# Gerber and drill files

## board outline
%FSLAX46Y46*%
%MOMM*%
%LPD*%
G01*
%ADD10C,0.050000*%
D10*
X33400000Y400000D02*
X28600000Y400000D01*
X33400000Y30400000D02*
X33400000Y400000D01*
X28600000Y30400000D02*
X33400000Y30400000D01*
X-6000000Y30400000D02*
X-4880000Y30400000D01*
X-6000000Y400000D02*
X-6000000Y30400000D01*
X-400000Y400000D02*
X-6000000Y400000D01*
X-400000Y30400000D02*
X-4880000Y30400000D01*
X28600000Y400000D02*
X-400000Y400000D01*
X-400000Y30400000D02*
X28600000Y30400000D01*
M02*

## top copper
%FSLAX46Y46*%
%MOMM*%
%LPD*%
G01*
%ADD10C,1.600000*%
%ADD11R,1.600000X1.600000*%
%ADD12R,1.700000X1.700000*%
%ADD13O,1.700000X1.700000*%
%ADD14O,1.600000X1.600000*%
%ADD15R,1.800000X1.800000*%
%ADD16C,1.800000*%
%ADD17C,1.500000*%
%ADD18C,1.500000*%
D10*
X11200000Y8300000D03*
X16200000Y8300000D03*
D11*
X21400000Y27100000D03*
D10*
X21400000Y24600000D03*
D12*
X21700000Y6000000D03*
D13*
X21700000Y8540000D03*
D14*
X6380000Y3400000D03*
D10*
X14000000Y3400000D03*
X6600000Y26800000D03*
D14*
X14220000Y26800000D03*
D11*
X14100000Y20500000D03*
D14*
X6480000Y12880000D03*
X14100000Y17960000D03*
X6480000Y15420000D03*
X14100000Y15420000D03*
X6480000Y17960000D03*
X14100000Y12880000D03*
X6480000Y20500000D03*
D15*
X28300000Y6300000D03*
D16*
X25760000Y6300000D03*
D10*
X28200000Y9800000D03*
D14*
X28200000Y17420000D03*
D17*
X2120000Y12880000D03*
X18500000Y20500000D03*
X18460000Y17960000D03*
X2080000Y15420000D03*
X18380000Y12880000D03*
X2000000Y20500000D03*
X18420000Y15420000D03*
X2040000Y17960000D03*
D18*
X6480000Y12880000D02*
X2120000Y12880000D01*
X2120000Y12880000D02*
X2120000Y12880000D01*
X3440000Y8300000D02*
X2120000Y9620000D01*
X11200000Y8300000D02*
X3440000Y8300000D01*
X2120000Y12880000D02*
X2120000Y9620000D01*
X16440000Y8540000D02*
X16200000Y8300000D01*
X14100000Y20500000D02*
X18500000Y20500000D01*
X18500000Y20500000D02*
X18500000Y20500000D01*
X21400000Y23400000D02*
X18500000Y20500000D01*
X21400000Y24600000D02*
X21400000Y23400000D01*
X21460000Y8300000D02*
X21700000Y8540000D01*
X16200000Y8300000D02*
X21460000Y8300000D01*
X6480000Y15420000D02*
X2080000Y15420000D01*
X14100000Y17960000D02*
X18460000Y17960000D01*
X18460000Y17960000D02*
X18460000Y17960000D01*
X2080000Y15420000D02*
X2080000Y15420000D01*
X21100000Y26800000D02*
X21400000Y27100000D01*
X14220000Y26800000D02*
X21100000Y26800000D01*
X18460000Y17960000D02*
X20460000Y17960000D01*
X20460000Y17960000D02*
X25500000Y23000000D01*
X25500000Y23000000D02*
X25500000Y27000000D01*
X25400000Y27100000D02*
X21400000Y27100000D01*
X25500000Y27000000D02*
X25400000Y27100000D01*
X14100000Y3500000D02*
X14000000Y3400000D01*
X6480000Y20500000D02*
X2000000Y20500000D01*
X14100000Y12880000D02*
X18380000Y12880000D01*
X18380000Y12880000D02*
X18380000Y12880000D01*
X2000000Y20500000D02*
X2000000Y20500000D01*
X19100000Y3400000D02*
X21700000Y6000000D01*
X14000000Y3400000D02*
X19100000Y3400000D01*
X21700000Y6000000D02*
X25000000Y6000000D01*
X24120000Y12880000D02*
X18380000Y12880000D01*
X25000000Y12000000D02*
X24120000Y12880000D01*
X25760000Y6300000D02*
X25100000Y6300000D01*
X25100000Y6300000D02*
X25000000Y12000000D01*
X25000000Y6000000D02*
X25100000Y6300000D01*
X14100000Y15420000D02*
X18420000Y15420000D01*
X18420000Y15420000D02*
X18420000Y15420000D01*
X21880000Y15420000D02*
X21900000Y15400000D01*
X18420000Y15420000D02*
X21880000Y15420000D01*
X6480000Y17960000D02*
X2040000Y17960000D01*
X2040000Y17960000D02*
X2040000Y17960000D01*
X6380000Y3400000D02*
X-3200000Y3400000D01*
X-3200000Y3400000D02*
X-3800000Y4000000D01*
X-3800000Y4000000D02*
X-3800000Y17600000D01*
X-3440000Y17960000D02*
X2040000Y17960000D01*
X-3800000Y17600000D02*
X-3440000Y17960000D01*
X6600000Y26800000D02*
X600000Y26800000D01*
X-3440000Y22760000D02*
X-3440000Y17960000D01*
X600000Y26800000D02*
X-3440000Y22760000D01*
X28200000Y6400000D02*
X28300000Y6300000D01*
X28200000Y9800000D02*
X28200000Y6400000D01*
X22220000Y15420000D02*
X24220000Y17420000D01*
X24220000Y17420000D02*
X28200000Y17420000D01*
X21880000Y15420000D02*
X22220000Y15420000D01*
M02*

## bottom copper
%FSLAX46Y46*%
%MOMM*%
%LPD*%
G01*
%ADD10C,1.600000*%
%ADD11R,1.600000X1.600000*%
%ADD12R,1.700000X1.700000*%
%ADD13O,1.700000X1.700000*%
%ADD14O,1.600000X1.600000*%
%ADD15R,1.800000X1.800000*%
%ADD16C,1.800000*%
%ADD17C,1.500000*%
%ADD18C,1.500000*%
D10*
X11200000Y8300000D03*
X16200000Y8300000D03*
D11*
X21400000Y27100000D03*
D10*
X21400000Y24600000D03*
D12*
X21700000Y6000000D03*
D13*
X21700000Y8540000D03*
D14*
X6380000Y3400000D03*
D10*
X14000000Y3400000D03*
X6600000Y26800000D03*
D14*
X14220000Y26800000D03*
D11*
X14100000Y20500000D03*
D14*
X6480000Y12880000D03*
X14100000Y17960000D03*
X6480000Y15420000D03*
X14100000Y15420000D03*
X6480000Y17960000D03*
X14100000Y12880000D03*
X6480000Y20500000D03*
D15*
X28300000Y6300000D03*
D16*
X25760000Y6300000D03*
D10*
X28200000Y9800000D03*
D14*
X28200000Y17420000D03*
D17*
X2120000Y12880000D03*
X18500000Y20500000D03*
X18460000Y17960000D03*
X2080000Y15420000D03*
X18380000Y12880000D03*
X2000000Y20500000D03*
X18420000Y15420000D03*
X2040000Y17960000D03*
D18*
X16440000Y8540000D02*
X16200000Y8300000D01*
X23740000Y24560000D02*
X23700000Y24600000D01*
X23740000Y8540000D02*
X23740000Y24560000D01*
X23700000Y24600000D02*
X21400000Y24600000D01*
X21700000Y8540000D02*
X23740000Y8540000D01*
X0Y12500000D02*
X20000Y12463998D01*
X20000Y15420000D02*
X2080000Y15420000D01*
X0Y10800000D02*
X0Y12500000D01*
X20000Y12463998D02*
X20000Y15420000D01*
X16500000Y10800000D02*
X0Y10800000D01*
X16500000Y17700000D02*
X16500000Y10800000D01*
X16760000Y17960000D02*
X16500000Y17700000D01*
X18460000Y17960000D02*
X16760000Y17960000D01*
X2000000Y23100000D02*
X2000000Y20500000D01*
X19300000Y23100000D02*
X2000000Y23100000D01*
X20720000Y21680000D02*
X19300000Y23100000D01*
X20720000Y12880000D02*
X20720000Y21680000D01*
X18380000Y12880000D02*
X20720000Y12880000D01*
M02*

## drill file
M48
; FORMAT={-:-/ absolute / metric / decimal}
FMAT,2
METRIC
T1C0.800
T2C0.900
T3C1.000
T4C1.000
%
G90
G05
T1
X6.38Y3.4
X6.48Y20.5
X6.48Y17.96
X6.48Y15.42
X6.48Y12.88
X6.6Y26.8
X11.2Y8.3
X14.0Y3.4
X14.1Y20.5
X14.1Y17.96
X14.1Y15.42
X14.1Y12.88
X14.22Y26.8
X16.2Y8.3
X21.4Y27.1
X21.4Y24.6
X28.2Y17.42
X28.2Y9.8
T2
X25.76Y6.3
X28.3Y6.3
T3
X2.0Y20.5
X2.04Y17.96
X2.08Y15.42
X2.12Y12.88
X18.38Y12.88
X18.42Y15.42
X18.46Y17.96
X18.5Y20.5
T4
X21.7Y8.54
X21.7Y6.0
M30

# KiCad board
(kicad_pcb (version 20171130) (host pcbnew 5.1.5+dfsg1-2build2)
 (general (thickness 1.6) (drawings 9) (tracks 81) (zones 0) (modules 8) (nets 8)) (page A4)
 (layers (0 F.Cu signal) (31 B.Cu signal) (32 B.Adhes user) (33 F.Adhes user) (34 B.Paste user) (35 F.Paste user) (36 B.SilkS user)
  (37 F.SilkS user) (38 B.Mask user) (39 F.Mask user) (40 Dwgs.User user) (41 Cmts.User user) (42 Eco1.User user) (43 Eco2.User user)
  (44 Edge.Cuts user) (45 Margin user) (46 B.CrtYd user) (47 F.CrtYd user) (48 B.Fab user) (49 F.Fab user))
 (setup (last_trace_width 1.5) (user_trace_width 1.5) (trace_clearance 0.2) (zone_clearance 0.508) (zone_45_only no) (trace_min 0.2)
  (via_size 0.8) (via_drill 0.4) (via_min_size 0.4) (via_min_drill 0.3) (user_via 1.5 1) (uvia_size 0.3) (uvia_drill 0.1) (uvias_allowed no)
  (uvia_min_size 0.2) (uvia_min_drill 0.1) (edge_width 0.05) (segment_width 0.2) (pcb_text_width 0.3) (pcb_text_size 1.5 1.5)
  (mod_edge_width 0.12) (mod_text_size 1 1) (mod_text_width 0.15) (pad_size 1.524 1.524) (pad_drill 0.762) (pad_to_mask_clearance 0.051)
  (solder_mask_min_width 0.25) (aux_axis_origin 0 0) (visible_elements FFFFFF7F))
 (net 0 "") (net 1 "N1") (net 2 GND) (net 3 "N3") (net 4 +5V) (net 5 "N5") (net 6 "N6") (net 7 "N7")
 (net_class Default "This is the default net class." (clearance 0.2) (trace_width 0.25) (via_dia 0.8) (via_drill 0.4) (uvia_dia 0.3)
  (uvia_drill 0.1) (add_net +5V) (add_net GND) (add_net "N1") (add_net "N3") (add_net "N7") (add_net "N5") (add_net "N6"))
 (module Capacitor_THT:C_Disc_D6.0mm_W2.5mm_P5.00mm (layer F.Cu) (at 11.2 -8.3)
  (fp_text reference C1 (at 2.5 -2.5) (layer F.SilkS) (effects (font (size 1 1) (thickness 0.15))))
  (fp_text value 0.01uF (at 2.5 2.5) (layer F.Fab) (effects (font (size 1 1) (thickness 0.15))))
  (pad 1 thru_hole circle (at 0 0) (size 1.6 1.6) (drill 0.8) (layers *.Cu *.Mask) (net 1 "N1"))
  (pad 2 thru_hole circle (at 5 0) (size 1.6 1.6) (drill 0.8) (layers *.Cu *.Mask) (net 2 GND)))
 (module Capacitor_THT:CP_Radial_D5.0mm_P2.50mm (layer F.Cu) (at 21.4 -27.1 270)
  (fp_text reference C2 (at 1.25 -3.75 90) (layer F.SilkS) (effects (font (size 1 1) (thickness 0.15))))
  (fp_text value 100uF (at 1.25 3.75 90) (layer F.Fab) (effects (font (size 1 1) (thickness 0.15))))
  (pad 1 thru_hole rect (at 0 0 270) (size 1.6 1.6) (drill 0.8) (layers *.Cu *.Mask) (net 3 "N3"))
  (pad 2 thru_hole circle (at 2.5 0 270) (size 1.6 1.6) (drill 0.8) (layers *.Cu *.Mask) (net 2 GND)))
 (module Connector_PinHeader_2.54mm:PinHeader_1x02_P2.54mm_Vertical (layer F.Cu) (at 21.7 -6 180)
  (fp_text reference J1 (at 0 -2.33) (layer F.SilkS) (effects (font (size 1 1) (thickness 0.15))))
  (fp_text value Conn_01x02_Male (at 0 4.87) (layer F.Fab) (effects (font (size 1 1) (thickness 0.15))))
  (pad 1 thru_hole rect (at 0 0 180) (size 1.7 1.7) (drill 1) (layers *.Cu *.Mask) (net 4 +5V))
  (pad 2 thru_hole oval (at 0 2.54 180) (size 1.7 1.7) (drill 1) (layers *.Cu *.Mask) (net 2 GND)))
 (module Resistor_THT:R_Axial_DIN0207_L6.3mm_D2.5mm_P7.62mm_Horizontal (layer F.Cu) (at 14 -3.4 180)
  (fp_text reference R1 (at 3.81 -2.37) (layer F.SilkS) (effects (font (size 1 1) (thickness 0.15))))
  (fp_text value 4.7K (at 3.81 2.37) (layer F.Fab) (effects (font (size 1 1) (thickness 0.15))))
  (pad 2 thru_hole oval (at 7.62 0 180) (size 1.6 1.6) (drill 0.8) (layers *.Cu *.Mask) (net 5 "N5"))
  (pad 1 thru_hole circle (at 0 0 180) (size 1.6 1.6) (drill 0.8) (layers *.Cu *.Mask) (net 4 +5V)))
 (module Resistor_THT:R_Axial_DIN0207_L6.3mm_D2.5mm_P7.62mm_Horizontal (layer F.Cu) (at 6.6 -26.8)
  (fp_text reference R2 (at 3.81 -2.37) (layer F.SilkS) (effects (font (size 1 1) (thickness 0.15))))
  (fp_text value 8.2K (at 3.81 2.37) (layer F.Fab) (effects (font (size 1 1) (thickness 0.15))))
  (pad 1 thru_hole circle (at 0 0) (size 1.6 1.6) (drill 0.8) (layers *.Cu *.Mask) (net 5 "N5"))
  (pad 2 thru_hole oval (at 7.62 0) (size 1.6 1.6) (drill 0.8) (layers *.Cu *.Mask) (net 3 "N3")))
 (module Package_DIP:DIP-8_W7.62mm (layer B.Cu) (at 14.1 -20.5 180)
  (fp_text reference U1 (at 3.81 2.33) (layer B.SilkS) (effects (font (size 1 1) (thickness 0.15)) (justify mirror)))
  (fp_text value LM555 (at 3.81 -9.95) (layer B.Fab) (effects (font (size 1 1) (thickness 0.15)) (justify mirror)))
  (pad 1 thru_hole rect (at 0 0 180) (size 1.6 1.6) (drill 0.8) (layers *.Cu *.Mask) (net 2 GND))
  (pad 5 thru_hole oval (at 7.62 -7.62 180) (size 1.6 1.6) (drill 0.8) (layers *.Cu *.Mask) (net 1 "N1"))
  (pad 2 thru_hole oval (at 0 -2.54 180) (size 1.6 1.6) (drill 0.8) (layers *.Cu *.Mask) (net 3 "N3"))
  (pad 6 thru_hole oval (at 7.62 -5.08 180) (size 1.6 1.6) (drill 0.8) (layers *.Cu *.Mask) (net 3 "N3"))
  (pad 3 thru_hole oval (at 0 -5.08 180) (size 1.6 1.6) (drill 0.8) (layers *.Cu *.Mask) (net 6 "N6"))
  (pad 7 thru_hole oval (at 7.62 -2.54 180) (size 1.6 1.6) (drill 0.8) (layers *.Cu *.Mask) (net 5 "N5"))
  (pad 4 thru_hole oval (at 0 -7.62 180) (size 1.6 1.6) (drill 0.8) (layers *.Cu *.Mask) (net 4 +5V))
  (pad 8 thru_hole oval (at 7.62 0 180) (size 1.6 1.6) (drill 0.8) (layers *.Cu *.Mask) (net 4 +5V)))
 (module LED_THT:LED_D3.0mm (layer F.Cu) (at 28.3 -6.3 180)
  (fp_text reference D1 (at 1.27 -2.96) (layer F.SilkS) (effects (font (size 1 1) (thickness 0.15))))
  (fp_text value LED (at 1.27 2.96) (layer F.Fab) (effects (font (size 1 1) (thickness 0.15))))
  (pad 1 thru_hole rect (at 0 0 180) (size 1.8 1.8) (drill 0.9) (layers *.Cu *.Mask) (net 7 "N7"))
  (pad 2 thru_hole circle (at 2.54 0 180) (size 1.8 1.8) (drill 0.9) (layers *.Cu *.Mask) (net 4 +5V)))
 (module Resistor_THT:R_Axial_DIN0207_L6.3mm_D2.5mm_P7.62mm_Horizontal (layer F.Cu) (at 28.2 -9.8 90)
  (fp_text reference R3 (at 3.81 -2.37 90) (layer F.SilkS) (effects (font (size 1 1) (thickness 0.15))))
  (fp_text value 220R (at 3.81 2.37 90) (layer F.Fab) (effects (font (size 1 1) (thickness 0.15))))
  (pad 1 thru_hole circle (at 0 0 90) (size 1.6 1.6) (drill 0.8) (layers *.Cu *.Mask) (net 7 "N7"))
  (pad 2 thru_hole oval (at 7.62 0 90) (size 1.6 1.6) (drill 0.8) (layers *.Cu *.Mask) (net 6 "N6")))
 (gr_line (start 33.4 -0.4) (end 28.6 -0.4) (layer Edge.Cuts) (width 0.05))
 (gr_line (start 33.4 -30.4) (end 33.4 -0.4) (layer Edge.Cuts) (width 0.05))
 (gr_line (start 28.6 -30.4) (end 33.4 -30.4) (layer Edge.Cuts) (width 0.05))
 (gr_line (start -6 -30.4) (end -4.88 -30.4) (layer Edge.Cuts) (width 0.05))
 (gr_line (start -6 -0.4) (end -6 -30.4) (layer Edge.Cuts) (width 0.05))
 (gr_line (start -0.4 -0.4) (end -6 -0.4) (layer Edge.Cuts) (width 0.05))
 (gr_line (start -0.4 -30.4) (end -4.88 -30.4) (layer Edge.Cuts) (width 0.05))
 (gr_line (start 28.6 -0.4) (end -0.4 -0.4) (layer Edge.Cuts) (width 0.05))
 (gr_line (start -0.4 -30.4) (end 28.6 -30.4) (layer Edge.Cuts) (width 0.05))
 (segment (start 6.48 -12.88) (end 2.12 -12.88) (width 1.5) (layer F.Cu) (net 1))
 (segment (start 2.12 -12.88) (end 2.12 -12.88) (width 1.5) (layer F.Cu) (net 1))
 (via (at 2.12 -12.88) (size 1.5) (drill 1) (layers F.Cu B.Cu) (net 1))
 (segment (start 3.44 -8.3) (end 2.12 -9.62) (width 1.5) (layer F.Cu) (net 1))
 (segment (start 11.2 -8.3) (end 3.44 -8.3) (width 1.5) (layer F.Cu) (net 1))
 (segment (start 2.12 -12.88) (end 2.12 -9.62) (width 1.5) (layer F.Cu) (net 1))
 (segment (start 16.44 -8.54) (end 16.2 -8.3) (width 1.5) (layer B.Cu) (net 2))
 (segment (start 16.44 -8.54) (end 16.2 -8.3) (width 1.5) (layer F.Cu) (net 2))
 (segment (start 14.1 -20.5) (end 18.5 -20.5) (width 1.5) (layer F.Cu) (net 2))
 (segment (start 18.5 -20.5) (end 18.5 -20.5) (width 1.5) (layer F.Cu) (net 2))
 (via (at 18.5 -20.5) (size 1.5) (drill 1) (layers F.Cu B.Cu) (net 2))
 (segment (start 21.4 -23.4) (end 18.5 -20.5) (width 1.5) (layer F.Cu) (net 2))
 (segment (start 21.4 -24.6) (end 21.4 -23.4) (width 1.5) (layer F.Cu) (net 2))
 (segment (start 21.46 -8.3) (end 21.7 -8.54) (width 1.5) (layer F.Cu) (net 2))
 (segment (start 16.2 -8.3) (end 21.46 -8.3) (width 1.5) (layer F.Cu) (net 2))
 (segment (start 23.74 -24.56) (end 23.7 -24.6) (width 1.5) (layer B.Cu) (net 2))
 (segment (start 23.74 -8.54) (end 23.74 -24.56) (width 1.5) (layer B.Cu) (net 2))
 (segment (start 23.7 -24.6) (end 21.4 -24.6) (width 1.5) (layer B.Cu) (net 2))
 (segment (start 21.7 -8.54) (end 23.74 -8.54) (width 1.5) (layer B.Cu) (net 2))
 (segment (start 6.48 -15.42) (end 2.08 -15.42) (width 1.5) (layer F.Cu) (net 3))
 (segment (start 14.1 -17.96) (end 18.46 -17.96) (width 1.5) (layer F.Cu) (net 3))
 (segment (start 18.46 -17.96) (end 18.46 -17.96) (width 1.5) (layer F.Cu) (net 3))
 (via (at 18.46 -17.96) (size 1.5) (drill 1) (layers F.Cu B.Cu) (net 3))
 (segment (start 2.08 -15.42) (end 2.08 -15.42) (width 1.5) (layer F.Cu) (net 3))
 (via (at 2.08 -15.42) (size 1.5) (drill 1) (layers F.Cu B.Cu) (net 3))
 (segment (start 21.1 -26.8) (end 21.4 -27.1) (width 1.5) (layer F.Cu) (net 3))
 (segment (start 14.22 -26.8) (end 21.1 -26.8) (width 1.5) (layer F.Cu) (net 3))
 (segment (start 18.46 -17.96) (end 20.46 -17.96) (width 1.5) (layer F.Cu) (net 3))
 (segment (start 20.46 -17.96) (end 25.5 -23) (width 1.5) (layer F.Cu) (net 3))
 (segment (start 25.5 -23) (end 25.5 -27) (width 1.5) (layer F.Cu) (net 3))
 (segment (start 25.4 -27.1) (end 21.4 -27.1) (width 1.5) (layer F.Cu) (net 3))
 (segment (start 25.5 -27) (end 25.4 -27.1) (width 1.5) (layer F.Cu) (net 3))
 (segment (start 0 -12.5) (end 0.02 -12.463998) (width 1.5) (layer B.Cu) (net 3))
 (segment (start 0.02 -15.42) (end 2.08 -15.42) (width 1.5) (layer B.Cu) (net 3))
 (segment (start 0 -10.8) (end 0 -12.5) (width 1.5) (layer B.Cu) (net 3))
 (segment (start 0.02 -12.463998) (end 0.02 -15.42) (width 1.5) (layer B.Cu) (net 3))
 (segment (start 16.5 -10.8) (end 0 -10.8) (width 1.5) (layer B.Cu) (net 3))
 (segment (start 16.5 -17.7) (end 16.5 -10.8) (width 1.5) (layer B.Cu) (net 3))
 (segment (start 16.76 -17.96) (end 16.5 -17.7) (width 1.5) (layer B.Cu) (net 3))
 (segment (start 18.46 -17.96) (end 16.76 -17.96) (width 1.5) (layer B.Cu) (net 3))
 (segment (start 14.1 -3.5) (end 14 -3.4) (width 1.5) (layer F.Cu) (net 4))
 (segment (start 6.48 -20.5) (end 2 -20.5) (width 1.5) (layer F.Cu) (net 4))
 (segment (start 14.1 -12.88) (end 18.38 -12.88) (width 1.5) (layer F.Cu) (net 4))
 (segment (start 18.38 -12.88) (end 18.38 -12.88) (width 1.5) (layer F.Cu) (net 4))
 (via (at 18.38 -12.88) (size 1.5) (drill 1) (layers F.Cu B.Cu) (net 4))
 (segment (start 2 -20.5) (end 2 -20.5) (width 1.5) (layer F.Cu) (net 4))
 (via (at 2 -20.5) (size 1.5) (drill 1) (layers F.Cu B.Cu) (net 4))
 (segment (start 19.1 -3.4) (end 21.7 -6) (width 1.5) (layer F.Cu) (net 4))
 (segment (start 14 -3.4) (end 19.1 -3.4) (width 1.5) (layer F.Cu) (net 4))
 (segment (start 21.7 -6) (end 25 -6) (width 1.5) (layer F.Cu) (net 4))
 (segment (start 24.12 -12.88) (end 18.38 -12.88) (width 1.5) (layer F.Cu) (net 4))
 (segment (start 25 -12) (end 24.12 -12.88) (width 1.5) (layer F.Cu) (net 4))
 (segment (start 2 -23.1) (end 2 -20.5) (width 1.5) (layer B.Cu) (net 4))
 (segment (start 19.3 -23.1) (end 2 -23.1) (width 1.5) (layer B.Cu) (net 4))
 (segment (start 20.72 -21.68) (end 19.3 -23.1) (width 1.5) (layer B.Cu) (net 4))
 (segment (start 20.72 -12.88) (end 20.72 -21.68) (width 1.5) (layer B.Cu) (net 4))
 (segment (start 18.38 -12.88) (end 20.72 -12.88) (width 1.5) (layer B.Cu) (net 4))
 (segment (start 25.76 -6.3) (end 25.1 -6.3) (width 1.5) (layer F.Cu) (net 4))
 (segment (start 25.1 -6.3) (end 25 -12) (width 1.5) (layer F.Cu) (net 4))
 (segment (start 25 -6) (end 25.1 -6.3) (width 1.5) (layer F.Cu) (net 4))
 (segment (start 14.1 -15.42) (end 18.42 -15.42) (width 1.5) (layer F.Cu) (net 6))
 (segment (start 18.42 -15.42) (end 18.42 -15.42) (width 1.5) (layer F.Cu) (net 6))
 (via (at 18.42 -15.42) (size 1.5) (drill 1) (layers F.Cu B.Cu) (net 6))
 (segment (start 21.88 -15.42) (end 21.9 -15.4) (width 1.5) (layer F.Cu) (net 6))
 (segment (start 18.42 -15.42) (end 21.88 -15.42) (width 1.5) (layer F.Cu) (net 6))
 (segment (start 6.48 -17.96) (end 2.04 -17.96) (width 1.5) (layer F.Cu) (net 5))
 (segment (start 2.04 -17.96) (end 2.04 -17.96) (width 1.5) (layer F.Cu) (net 5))
 (via (at 2.04 -17.96) (size 1.5) (drill 1) (layers F.Cu B.Cu) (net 5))
 (segment (start 6.38 -3.4) (end -3.2 -3.4) (width 1.5) (layer F.Cu) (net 5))
 (segment (start -3.2 -3.4) (end -3.8 -4) (width 1.5) (layer F.Cu) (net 5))
 (segment (start -3.8 -4) (end -3.8 -17.6) (width 1.5) (layer F.Cu) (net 5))
 (segment (start -3.44 -17.96) (end 2.04 -17.96) (width 1.5) (layer F.Cu) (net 5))
 (segment (start -3.8 -17.6) (end -3.44 -17.96) (width 1.5) (layer F.Cu) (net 5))
 (segment (start 6.6 -26.8) (end 0.6 -26.8) (width 1.5) (layer F.Cu) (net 5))
 (segment (start -3.44 -22.76) (end -3.44 -17.96) (width 1.5) (layer F.Cu) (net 5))
 (segment (start 0.6 -26.8) (end -3.44 -22.76) (width 1.5) (layer F.Cu) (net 5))
 (segment (start 28.2 -6.4) (end 28.3 -6.3) (width 1.5) (layer F.Cu) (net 7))
 (segment (start 28.2 -9.8) (end 28.2 -6.4) (width 1.5) (layer F.Cu) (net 7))
 (segment (start 22.22 -15.42) (end 24.22 -17.42) (width 1.5) (layer F.Cu) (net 6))
 (segment (start 24.22 -17.42) (end 28.2 -17.42) (width 1.5) (layer F.Cu) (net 6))
 (segment (start 21.88 -15.42) (end 22.22 -15.42) (width 1.5) (layer F.Cu) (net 6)))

